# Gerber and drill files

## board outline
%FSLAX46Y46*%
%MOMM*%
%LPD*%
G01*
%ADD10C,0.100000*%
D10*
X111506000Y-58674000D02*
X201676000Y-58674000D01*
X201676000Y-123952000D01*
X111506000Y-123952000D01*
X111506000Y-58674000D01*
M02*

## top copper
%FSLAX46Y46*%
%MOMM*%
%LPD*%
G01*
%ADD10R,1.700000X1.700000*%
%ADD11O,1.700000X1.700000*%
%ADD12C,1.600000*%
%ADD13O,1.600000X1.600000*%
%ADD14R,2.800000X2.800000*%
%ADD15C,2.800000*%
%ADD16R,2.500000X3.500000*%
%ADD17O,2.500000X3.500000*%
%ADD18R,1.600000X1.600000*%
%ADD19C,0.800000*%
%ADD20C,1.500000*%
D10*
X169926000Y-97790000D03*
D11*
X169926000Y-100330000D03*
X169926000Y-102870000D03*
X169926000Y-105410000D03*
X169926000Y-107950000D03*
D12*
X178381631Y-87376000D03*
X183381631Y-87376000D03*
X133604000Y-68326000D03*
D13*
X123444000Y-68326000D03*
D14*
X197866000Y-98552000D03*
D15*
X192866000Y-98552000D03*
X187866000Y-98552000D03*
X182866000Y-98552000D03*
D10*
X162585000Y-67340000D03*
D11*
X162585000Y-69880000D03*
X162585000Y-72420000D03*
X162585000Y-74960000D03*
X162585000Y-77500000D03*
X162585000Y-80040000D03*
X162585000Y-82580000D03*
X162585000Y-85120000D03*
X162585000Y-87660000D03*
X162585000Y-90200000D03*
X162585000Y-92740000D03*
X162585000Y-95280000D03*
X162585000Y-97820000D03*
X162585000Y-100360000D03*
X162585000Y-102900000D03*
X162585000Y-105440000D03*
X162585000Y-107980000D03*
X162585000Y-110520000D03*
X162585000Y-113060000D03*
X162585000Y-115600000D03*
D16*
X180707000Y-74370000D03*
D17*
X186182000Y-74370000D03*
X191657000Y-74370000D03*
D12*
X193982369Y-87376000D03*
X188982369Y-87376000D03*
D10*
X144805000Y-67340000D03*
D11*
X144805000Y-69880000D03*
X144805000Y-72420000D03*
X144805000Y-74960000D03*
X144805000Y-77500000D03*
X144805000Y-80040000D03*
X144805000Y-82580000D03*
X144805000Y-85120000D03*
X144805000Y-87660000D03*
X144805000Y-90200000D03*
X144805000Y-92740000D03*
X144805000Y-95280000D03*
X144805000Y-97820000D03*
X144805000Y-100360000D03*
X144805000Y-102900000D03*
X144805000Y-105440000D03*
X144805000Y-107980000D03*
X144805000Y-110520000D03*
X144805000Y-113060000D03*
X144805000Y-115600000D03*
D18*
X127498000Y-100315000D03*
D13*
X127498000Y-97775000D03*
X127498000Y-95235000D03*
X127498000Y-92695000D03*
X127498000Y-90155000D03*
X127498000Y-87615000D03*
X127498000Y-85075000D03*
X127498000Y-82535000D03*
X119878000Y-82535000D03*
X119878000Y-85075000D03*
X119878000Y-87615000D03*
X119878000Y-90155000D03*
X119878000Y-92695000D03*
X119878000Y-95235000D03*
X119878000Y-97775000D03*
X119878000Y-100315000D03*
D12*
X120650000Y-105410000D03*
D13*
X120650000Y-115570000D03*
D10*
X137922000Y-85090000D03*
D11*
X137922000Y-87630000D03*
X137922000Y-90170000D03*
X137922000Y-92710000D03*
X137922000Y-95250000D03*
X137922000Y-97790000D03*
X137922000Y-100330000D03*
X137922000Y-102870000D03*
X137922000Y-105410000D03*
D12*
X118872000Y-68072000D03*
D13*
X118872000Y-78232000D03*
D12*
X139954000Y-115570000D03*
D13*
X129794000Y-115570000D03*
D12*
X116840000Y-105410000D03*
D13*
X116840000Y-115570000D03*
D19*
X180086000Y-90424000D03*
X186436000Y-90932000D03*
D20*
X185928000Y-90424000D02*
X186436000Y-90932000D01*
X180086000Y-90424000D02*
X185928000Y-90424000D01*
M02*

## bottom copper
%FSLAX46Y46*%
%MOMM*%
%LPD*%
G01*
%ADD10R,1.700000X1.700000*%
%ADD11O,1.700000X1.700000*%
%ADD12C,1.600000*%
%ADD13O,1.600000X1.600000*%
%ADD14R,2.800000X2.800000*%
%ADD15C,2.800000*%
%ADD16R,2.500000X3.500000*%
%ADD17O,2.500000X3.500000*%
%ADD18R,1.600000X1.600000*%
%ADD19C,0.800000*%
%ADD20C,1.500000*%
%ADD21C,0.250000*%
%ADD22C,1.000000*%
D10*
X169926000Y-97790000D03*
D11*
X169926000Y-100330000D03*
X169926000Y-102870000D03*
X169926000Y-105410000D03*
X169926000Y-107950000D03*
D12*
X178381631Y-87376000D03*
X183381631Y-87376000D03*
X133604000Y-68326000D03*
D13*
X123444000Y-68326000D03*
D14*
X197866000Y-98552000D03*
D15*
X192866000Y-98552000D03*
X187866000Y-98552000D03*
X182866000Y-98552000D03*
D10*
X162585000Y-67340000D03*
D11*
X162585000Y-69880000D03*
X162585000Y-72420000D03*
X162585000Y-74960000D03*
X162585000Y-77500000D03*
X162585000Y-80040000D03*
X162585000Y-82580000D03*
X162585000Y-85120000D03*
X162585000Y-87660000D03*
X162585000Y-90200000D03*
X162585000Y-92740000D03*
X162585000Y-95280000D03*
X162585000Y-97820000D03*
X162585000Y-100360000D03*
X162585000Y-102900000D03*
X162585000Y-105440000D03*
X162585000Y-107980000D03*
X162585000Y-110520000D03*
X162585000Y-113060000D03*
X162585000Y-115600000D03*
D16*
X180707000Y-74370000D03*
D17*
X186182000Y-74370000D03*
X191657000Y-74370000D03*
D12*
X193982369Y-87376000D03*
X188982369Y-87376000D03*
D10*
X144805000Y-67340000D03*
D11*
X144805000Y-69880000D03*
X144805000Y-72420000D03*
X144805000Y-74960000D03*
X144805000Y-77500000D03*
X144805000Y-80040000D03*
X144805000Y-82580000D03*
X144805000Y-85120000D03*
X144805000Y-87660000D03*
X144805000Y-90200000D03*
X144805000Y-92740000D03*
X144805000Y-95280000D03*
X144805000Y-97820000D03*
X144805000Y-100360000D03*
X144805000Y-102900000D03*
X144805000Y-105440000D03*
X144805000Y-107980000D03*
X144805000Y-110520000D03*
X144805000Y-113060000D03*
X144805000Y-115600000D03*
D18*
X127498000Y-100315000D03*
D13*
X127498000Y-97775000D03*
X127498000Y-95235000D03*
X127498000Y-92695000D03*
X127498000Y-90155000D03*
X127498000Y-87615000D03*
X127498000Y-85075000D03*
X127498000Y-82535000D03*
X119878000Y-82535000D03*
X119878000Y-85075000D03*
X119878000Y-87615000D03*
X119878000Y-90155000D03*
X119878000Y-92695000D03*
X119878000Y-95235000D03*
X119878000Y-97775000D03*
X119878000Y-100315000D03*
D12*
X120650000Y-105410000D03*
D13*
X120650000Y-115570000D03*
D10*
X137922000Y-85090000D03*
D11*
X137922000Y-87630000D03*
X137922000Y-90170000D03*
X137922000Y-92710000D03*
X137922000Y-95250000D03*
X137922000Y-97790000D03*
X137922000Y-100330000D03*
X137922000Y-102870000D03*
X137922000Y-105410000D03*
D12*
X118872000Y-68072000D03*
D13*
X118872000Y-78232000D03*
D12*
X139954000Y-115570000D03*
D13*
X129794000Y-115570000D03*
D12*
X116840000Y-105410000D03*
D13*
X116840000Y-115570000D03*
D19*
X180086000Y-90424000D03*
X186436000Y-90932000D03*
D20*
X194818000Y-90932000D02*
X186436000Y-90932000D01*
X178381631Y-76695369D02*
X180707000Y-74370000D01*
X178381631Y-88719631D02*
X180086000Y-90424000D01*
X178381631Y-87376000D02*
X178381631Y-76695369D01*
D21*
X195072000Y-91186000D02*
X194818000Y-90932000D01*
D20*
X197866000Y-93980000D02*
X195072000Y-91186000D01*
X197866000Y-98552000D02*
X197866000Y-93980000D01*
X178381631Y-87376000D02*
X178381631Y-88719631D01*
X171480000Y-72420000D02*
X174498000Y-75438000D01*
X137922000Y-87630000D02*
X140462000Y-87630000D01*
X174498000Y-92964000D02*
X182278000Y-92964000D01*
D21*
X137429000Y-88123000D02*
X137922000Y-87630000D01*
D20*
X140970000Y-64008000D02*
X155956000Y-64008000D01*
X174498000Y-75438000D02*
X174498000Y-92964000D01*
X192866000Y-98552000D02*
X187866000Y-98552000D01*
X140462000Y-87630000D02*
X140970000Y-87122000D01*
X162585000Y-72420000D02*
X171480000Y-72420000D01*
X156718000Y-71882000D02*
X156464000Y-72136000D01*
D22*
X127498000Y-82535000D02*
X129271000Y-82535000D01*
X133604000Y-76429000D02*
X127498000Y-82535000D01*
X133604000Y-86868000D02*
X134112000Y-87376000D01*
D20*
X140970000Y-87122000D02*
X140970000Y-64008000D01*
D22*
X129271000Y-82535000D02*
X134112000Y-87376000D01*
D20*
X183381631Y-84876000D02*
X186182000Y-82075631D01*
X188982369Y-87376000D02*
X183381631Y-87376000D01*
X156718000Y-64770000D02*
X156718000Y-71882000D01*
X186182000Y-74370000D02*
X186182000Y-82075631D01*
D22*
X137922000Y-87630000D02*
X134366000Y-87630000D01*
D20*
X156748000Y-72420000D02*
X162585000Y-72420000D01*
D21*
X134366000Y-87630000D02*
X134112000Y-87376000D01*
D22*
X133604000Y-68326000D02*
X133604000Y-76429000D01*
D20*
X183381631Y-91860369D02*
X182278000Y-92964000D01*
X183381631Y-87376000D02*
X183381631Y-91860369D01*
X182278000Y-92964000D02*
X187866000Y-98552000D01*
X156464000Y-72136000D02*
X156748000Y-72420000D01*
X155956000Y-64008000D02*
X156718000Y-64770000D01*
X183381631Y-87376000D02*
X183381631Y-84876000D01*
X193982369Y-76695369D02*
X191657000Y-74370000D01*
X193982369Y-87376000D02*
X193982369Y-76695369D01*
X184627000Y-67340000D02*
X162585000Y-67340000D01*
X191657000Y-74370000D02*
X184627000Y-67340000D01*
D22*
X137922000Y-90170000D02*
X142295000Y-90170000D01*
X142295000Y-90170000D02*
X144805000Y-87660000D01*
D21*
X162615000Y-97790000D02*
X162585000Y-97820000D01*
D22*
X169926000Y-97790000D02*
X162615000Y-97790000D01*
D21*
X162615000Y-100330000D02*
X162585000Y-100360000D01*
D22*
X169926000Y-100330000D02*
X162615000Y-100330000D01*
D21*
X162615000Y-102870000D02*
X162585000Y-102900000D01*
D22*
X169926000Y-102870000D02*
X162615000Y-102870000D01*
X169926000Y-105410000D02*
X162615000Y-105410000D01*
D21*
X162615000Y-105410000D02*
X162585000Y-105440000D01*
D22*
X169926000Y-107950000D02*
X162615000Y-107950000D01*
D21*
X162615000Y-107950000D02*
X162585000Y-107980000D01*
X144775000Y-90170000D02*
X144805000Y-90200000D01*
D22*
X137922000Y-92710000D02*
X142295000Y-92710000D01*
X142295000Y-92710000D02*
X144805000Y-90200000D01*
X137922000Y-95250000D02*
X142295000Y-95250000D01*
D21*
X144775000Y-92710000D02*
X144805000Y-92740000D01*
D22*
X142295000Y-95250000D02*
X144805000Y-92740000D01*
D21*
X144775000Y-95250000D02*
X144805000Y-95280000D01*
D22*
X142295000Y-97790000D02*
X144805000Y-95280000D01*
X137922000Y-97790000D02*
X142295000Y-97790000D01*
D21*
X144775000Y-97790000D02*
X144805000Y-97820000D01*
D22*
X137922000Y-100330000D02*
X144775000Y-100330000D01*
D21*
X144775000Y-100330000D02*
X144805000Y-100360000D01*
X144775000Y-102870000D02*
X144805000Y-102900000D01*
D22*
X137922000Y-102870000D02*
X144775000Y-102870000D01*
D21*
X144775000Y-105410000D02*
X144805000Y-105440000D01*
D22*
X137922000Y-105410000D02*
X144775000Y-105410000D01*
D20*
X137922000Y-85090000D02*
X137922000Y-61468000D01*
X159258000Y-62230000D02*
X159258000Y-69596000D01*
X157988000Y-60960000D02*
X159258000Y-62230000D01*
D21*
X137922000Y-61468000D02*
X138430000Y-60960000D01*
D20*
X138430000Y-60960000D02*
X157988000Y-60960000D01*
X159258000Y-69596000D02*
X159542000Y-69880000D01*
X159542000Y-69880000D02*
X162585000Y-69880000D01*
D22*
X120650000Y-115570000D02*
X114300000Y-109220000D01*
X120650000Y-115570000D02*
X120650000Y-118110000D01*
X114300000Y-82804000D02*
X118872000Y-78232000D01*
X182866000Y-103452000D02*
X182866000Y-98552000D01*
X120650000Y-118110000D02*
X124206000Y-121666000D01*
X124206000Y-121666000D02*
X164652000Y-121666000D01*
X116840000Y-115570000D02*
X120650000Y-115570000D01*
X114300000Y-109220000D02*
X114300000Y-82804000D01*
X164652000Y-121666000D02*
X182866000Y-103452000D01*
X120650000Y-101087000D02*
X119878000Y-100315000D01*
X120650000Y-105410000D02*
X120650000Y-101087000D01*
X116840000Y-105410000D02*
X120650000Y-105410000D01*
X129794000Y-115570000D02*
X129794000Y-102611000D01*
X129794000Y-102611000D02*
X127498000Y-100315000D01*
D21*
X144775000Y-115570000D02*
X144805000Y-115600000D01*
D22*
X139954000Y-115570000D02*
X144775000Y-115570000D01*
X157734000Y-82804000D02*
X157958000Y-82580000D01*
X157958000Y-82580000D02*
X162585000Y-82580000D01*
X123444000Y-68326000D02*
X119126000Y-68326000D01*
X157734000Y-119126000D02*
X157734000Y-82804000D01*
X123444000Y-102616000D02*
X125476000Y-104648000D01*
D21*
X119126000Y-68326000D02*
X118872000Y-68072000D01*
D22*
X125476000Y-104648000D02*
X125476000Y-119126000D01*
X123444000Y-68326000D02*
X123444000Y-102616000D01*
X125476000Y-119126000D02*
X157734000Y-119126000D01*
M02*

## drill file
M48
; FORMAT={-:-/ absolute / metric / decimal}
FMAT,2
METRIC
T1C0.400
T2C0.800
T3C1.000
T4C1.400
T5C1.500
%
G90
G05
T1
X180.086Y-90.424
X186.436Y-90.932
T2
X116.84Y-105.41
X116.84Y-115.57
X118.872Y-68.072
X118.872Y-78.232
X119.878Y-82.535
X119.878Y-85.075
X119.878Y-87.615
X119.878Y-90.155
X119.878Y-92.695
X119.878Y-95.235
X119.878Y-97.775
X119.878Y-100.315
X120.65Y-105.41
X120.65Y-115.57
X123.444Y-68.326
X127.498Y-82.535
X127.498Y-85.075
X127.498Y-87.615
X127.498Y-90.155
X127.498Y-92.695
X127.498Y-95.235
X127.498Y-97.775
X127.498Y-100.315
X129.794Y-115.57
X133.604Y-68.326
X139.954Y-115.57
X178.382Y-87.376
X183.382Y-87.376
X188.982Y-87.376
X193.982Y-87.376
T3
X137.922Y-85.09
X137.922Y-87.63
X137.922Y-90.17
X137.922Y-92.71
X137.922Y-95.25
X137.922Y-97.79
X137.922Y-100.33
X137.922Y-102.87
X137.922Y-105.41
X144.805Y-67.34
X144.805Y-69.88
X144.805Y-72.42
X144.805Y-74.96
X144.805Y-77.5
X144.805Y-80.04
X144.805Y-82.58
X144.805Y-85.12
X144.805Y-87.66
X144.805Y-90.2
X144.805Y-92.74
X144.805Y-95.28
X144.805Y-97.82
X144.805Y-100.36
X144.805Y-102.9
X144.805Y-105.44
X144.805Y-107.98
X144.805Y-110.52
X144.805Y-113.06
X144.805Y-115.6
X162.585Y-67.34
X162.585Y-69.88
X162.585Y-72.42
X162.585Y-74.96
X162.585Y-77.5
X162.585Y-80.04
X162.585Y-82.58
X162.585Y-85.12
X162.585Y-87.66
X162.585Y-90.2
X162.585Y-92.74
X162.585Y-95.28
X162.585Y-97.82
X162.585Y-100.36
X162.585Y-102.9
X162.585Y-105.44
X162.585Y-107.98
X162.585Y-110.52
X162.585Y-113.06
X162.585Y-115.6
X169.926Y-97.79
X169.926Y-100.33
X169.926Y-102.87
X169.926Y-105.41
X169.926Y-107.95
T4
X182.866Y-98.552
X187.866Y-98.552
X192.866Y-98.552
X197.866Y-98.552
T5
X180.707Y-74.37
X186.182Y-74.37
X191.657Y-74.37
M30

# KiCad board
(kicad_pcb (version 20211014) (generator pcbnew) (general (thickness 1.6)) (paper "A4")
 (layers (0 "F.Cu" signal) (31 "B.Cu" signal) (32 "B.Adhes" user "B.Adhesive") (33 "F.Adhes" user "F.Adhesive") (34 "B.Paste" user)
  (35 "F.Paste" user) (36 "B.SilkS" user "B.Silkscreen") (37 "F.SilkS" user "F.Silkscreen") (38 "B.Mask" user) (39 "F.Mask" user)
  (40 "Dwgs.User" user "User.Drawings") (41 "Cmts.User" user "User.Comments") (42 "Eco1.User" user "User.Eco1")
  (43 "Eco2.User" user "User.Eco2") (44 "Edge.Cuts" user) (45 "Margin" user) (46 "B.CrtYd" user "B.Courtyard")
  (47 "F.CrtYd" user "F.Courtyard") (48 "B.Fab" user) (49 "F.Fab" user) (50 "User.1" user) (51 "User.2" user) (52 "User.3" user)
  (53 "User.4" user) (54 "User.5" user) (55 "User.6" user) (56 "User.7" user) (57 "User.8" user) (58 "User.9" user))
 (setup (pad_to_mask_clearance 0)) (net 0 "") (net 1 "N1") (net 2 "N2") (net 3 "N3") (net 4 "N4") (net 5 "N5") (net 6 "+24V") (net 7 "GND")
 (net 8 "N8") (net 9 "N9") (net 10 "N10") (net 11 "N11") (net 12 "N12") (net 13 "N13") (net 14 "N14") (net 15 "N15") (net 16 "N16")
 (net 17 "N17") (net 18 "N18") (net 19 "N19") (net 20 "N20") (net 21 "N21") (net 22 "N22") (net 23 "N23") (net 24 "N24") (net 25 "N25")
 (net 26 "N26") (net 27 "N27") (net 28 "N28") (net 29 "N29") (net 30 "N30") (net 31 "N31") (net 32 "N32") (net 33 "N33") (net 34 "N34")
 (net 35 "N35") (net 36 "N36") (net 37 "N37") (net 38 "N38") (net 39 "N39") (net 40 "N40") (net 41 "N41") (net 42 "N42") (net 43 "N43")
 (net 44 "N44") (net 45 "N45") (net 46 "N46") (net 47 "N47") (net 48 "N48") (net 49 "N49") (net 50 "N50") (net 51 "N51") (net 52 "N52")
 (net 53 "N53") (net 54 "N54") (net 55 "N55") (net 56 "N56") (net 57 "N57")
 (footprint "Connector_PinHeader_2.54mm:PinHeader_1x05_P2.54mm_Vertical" (layer "F.Cu") (at 169.926 97.79)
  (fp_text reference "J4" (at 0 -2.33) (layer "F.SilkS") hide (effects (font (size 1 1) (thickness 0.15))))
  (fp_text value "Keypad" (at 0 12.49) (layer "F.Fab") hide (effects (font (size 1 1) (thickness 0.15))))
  (pad "1" thru_hole rect (at 0 0) (size 1.7 1.7) (drill 1) (layers *.Cu *.Mask) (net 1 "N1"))
  (pad "2" thru_hole oval (at 0 2.54) (size 1.7 1.7) (drill 1) (layers *.Cu *.Mask) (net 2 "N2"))
  (pad "3" thru_hole oval (at 0 5.08) (size 1.7 1.7) (drill 1) (layers *.Cu *.Mask) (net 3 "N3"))
  (pad "4" thru_hole oval (at 0 7.62) (size 1.7 1.7) (drill 1) (layers *.Cu *.Mask) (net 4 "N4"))
  (pad "5" thru_hole oval (at 0 10.16) (size 1.7 1.7) (drill 1) (layers *.Cu *.Mask) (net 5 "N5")))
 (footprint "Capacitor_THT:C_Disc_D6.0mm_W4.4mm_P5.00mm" (layer "F.Cu") (at 178.381631 87.376)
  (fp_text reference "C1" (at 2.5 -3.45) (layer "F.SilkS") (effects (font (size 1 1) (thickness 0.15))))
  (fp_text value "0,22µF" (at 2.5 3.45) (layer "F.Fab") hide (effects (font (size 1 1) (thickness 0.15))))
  (pad "1" thru_hole circle (at 0 0) (size 1.6 1.6) (drill 0.8) (layers *.Cu *.Mask) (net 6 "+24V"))
  (pad "2" thru_hole circle (at 5 0) (size 1.6 1.6) (drill 0.8) (layers *.Cu *.Mask) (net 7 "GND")))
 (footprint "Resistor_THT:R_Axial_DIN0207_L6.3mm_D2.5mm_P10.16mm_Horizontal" (layer "F.Cu") (at 133.604 68.326 180)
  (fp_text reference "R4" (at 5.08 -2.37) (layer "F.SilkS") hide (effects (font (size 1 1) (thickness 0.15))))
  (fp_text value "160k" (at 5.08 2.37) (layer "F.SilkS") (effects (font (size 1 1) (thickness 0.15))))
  (pad "1" thru_hole circle (at 0 0 180) (size 1.6 1.6) (drill 0.8) (layers *.Cu *.Mask) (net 7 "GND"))
  (pad "2" thru_hole oval (at 10.16 0 180) (size 1.6 1.6) (drill 0.8) (layers *.Cu *.Mask) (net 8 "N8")))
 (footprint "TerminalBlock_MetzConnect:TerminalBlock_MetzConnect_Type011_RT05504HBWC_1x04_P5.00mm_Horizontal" (layer "F.Cu")
  (at 197.866 98.552 180)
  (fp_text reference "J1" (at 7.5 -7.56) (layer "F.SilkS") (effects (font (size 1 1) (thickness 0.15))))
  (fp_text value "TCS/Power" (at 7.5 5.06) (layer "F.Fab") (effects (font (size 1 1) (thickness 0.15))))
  (pad "1" thru_hole rect (at 0 0 180) (size 2.8 2.8) (drill 1.4) (layers *.Cu *.Mask) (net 6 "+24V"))
  (pad "2" thru_hole circle (at 5 0 180) (size 2.8 2.8) (drill 1.4) (layers *.Cu *.Mask) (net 7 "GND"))
  (pad "3" thru_hole circle (at 10 0 180) (size 2.8 2.8) (drill 1.4) (layers *.Cu *.Mask) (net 7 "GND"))
  (pad "4" thru_hole circle (at 15 0 180) (size 2.8 2.8) (drill 1.4) (layers *.Cu *.Mask) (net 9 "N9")))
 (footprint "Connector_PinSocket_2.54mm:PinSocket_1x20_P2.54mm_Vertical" (layer "F.Cu") (at 162.585 67.34)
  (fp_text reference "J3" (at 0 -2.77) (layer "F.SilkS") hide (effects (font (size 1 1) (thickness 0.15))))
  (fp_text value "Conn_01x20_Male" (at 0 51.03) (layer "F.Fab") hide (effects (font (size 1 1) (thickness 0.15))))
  (pad "1" thru_hole rect (at 0 0) (size 1.7 1.7) (drill 1) (layers *.Cu *.Mask) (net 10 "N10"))
  (pad "2" thru_hole oval (at 0 2.54) (size 1.7 1.7) (drill 1) (layers *.Cu *.Mask) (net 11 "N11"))
  (pad "3" thru_hole oval (at 0 5.08) (size 1.7 1.7) (drill 1) (layers *.Cu *.Mask) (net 7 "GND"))
  (pad "4" thru_hole oval (at 0 7.62) (size 1.7 1.7) (drill 1) (layers *.Cu *.Mask) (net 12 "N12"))
  (pad "5" thru_hole oval (at 0 10.16) (size 1.7 1.7) (drill 1) (layers *.Cu *.Mask) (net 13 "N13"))
  (pad "6" thru_hole oval (at 0 12.7) (size 1.7 1.7) (drill 1) (layers *.Cu *.Mask) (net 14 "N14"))
  (pad "7" thru_hole oval (at 0 15.24) (size 1.7 1.7) (drill 1) (layers *.Cu *.Mask) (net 8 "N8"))
  (pad "8" thru_hole oval (at 0 17.78) (size 1.7 1.7) (drill 1) (layers *.Cu *.Mask) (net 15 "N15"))
  (pad "9" thru_hole oval (at 0 20.32) (size 1.7 1.7) (drill 1) (layers *.Cu *.Mask) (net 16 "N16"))
  (pad "10" thru_hole oval (at 0 22.86) (size 1.7 1.7) (drill 1) (layers *.Cu *.Mask) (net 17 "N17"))
  (pad "11" thru_hole oval (at 0 25.4) (size 1.7 1.7) (drill 1) (layers *.Cu *.Mask) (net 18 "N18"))
  (pad "12" thru_hole oval (at 0 27.94) (size 1.7 1.7) (drill 1) (layers *.Cu *.Mask) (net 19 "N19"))
  (pad "13" thru_hole oval (at 0 30.48) (size 1.7 1.7) (drill 1) (layers *.Cu *.Mask) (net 1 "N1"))
  (pad "14" thru_hole oval (at 0 33.02) (size 1.7 1.7) (drill 1) (layers *.Cu *.Mask) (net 2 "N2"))
  (pad "15" thru_hole oval (at 0 35.56) (size 1.7 1.7) (drill 1) (layers *.Cu *.Mask) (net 3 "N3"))
  (pad "16" thru_hole oval (at 0 38.1) (size 1.7 1.7) (drill 1) (layers *.Cu *.Mask) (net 4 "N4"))
  (pad "17" thru_hole oval (at 0 40.64) (size 1.7 1.7) (drill 1) (layers *.Cu *.Mask) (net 5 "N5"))
  (pad "18" thru_hole oval (at 0 43.18) (size 1.7 1.7) (drill 1) (layers *.Cu *.Mask) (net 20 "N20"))
  (pad "19" thru_hole oval (at 0 45.72) (size 1.7 1.7) (drill 1) (layers *.Cu *.Mask) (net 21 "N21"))
  (pad "20" thru_hole oval (at 0 48.26) (size 1.7 1.7) (drill 1) (layers *.Cu *.Mask) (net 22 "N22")))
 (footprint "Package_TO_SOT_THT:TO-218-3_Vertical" (layer "F.Cu") (at 180.707 74.37)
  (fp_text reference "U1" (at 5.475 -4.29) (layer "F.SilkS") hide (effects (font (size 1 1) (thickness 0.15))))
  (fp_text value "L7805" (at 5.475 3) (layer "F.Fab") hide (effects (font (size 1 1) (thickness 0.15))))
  (pad "1" thru_hole rect (at 0 0) (size 2.5 3.5) (drill 1.5) (layers *.Cu *.Mask) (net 6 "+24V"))
  (pad "2" thru_hole oval (at 5.475 0) (size 2.5 3.5) (drill 1.5) (layers *.Cu *.Mask) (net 7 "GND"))
  (pad "3" thru_hole oval (at 10.95 0) (size 2.5 3.5) (drill 1.5) (layers *.Cu *.Mask) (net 10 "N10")))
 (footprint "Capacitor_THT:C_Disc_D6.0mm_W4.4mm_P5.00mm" (layer "F.Cu") (at 193.982369 87.376 180)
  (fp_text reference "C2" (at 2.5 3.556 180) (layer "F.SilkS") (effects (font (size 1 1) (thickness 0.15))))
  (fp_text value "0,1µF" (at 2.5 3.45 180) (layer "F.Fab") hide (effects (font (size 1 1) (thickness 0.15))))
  (pad "1" thru_hole circle (at 0 0 180) (size 1.6 1.6) (drill 0.8) (layers *.Cu *.Mask) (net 10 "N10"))
  (pad "2" thru_hole circle (at 5 0 180) (size 1.6 1.6) (drill 0.8) (layers *.Cu *.Mask) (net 7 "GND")))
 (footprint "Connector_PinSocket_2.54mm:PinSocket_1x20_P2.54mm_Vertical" (layer "F.Cu") (at 144.805 67.34)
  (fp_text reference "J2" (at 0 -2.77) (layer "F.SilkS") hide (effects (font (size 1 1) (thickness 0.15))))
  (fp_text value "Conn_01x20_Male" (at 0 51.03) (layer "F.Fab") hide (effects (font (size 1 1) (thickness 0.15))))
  (pad "1" thru_hole rect (at 0 0) (size 1.7 1.7) (drill 1) (layers *.Cu *.Mask) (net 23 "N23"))
  (pad "2" thru_hole oval (at 0 2.54) (size 1.7 1.7) (drill 1) (layers *.Cu *.Mask) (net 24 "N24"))
  (pad "3" thru_hole oval (at 0 5.08) (size 1.7 1.7) (drill 1) (layers *.Cu *.Mask) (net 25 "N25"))
  (pad "4" thru_hole oval (at 0 7.62) (size 1.7 1.7) (drill 1) (layers *.Cu *.Mask) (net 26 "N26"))
  (pad "5" thru_hole oval (at 0 10.16) (size 1.7 1.7) (drill 1) (layers *.Cu *.Mask) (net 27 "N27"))
  (pad "6" thru_hole oval (at 0 12.7) (size 1.7 1.7) (drill 1) (layers *.Cu *.Mask) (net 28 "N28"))
  (pad "7" thru_hole oval (at 0 15.24) (size 1.7 1.7) (drill 1) (layers *.Cu *.Mask) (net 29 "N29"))
  (pad "8" thru_hole oval (at 0 17.78) (size 1.7 1.7) (drill 1) (layers *.Cu *.Mask) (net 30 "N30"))
  (pad "9" thru_hole oval (at 0 20.32) (size 1.7 1.7) (drill 1) (layers *.Cu *.Mask) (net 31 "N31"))
  (pad "10" thru_hole oval (at 0 22.86) (size 1.7 1.7) (drill 1) (layers *.Cu *.Mask) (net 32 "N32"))
  (pad "11" thru_hole oval (at 0 25.4) (size 1.7 1.7) (drill 1) (layers *.Cu *.Mask) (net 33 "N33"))
  (pad "12" thru_hole oval (at 0 27.94) (size 1.7 1.7) (drill 1) (layers *.Cu *.Mask) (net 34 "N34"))
  (pad "13" thru_hole oval (at 0 30.48) (size 1.7 1.7) (drill 1) (layers *.Cu *.Mask) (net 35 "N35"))
  (pad "14" thru_hole oval (at 0 33.02) (size 1.7 1.7) (drill 1) (layers *.Cu *.Mask) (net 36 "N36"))
  (pad "15" thru_hole oval (at 0 35.56) (size 1.7 1.7) (drill 1) (layers *.Cu *.Mask) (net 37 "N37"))
  (pad "16" thru_hole oval (at 0 38.1) (size 1.7 1.7) (drill 1) (layers *.Cu *.Mask) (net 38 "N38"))
  (pad "17" thru_hole oval (at 0 40.64) (size 1.7 1.7) (drill 1) (layers *.Cu *.Mask) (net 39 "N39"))
  (pad "18" thru_hole oval (at 0 43.18) (size 1.7 1.7) (drill 1) (layers *.Cu *.Mask) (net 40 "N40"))
  (pad "19" thru_hole oval (at 0 45.72) (size 1.7 1.7) (drill 1) (layers *.Cu *.Mask) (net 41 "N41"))
  (pad "20" thru_hole oval (at 0 48.26) (size 1.7 1.7) (drill 1) (layers *.Cu *.Mask) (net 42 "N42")))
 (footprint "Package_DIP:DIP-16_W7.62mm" (layer "F.Cu") (at 127.498 100.315 180)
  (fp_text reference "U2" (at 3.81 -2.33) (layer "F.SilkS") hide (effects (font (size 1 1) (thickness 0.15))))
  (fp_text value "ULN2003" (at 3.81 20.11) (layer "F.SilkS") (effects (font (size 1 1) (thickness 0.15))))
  (pad "1" thru_hole rect (at 0 0 180) (size 1.6 1.6) (drill 0.8) (layers *.Cu *.Mask) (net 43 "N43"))
  (pad "2" thru_hole oval (at 0 2.54 180) (size 1.6 1.6) (drill 0.8) (layers *.Cu *.Mask) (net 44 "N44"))
  (pad "3" thru_hole oval (at 0 5.08 180) (size 1.6 1.6) (drill 0.8) (layers *.Cu *.Mask) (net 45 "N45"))
  (pad "4" thru_hole oval (at 0 7.62 180) (size 1.6 1.6) (drill 0.8) (layers *.Cu *.Mask) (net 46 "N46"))
  (pad "5" thru_hole oval (at 0 10.16 180) (size 1.6 1.6) (drill 0.8) (layers *.Cu *.Mask) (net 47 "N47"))
  (pad "6" thru_hole oval (at 0 12.7 180) (size 1.6 1.6) (drill 0.8) (layers *.Cu *.Mask) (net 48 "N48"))
  (pad "7" thru_hole oval (at 0 15.24 180) (size 1.6 1.6) (drill 0.8) (layers *.Cu *.Mask) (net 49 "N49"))
  (pad "8" thru_hole oval (at 0 17.78 180) (size 1.6 1.6) (drill 0.8) (layers *.Cu *.Mask) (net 7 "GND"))
  (pad "9" thru_hole oval (at 7.62 17.78 180) (size 1.6 1.6) (drill 0.8) (layers *.Cu *.Mask) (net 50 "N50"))
  (pad "10" thru_hole oval (at 7.62 15.24 180) (size 1.6 1.6) (drill 0.8) (layers *.Cu *.Mask) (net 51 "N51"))
  (pad "11" thru_hole oval (at 7.62 12.7 180) (size 1.6 1.6) (drill 0.8) (layers *.Cu *.Mask) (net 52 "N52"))
  (pad "12" thru_hole oval (at 7.62 10.16 180) (size 1.6 1.6) (drill 0.8) (layers *.Cu *.Mask) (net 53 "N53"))
  (pad "13" thru_hole oval (at 7.62 7.62 180) (size 1.6 1.6) (drill 0.8) (layers *.Cu *.Mask) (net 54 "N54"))
  (pad "14" thru_hole oval (at 7.62 5.08 180) (size 1.6 1.6) (drill 0.8) (layers *.Cu *.Mask) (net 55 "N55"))
  (pad "15" thru_hole oval (at 7.62 2.54 180) (size 1.6 1.6) (drill 0.8) (layers *.Cu *.Mask) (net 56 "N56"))
  (pad "16" thru_hole oval (at 7.62 0 180) (size 1.6 1.6) (drill 0.8) (layers *.Cu *.Mask) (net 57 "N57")))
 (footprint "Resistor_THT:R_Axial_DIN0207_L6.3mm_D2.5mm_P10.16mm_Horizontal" (layer "F.Cu") (at 120.65 105.41 -90)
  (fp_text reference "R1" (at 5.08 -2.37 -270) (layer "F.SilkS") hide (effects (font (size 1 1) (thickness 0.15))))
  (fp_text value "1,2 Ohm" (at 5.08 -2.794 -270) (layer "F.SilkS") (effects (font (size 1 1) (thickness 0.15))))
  (pad "1" thru_hole circle (at 0 0 270) (size 1.6 1.6) (drill 0.8) (layers *.Cu *.Mask) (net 57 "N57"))
  (pad "2" thru_hole oval (at 10.16 0 270) (size 1.6 1.6) (drill 0.8) (layers *.Cu *.Mask) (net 9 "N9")))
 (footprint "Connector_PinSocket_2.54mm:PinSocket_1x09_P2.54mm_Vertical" (layer "F.Cu") (at 137.922 85.09)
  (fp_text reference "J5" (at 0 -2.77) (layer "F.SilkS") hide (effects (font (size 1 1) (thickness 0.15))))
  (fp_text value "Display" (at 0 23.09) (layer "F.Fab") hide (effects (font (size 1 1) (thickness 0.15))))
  (pad "1" thru_hole rect (at 0 0) (size 1.7 1.7) (drill 1) (layers *.Cu *.Mask) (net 11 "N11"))
  (pad "2" thru_hole oval (at 0 2.54) (size 1.7 1.7) (drill 1) (layers *.Cu *.Mask) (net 7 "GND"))
  (pad "3" thru_hole oval (at 0 5.08) (size 1.7 1.7) (drill 1) (layers *.Cu *.Mask) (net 31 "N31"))
  (pad "4" thru_hole oval (at 0 7.62) (size 1.7 1.7) (drill 1) (layers *.Cu *.Mask) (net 32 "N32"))
  (pad "5" thru_hole oval (at 0 10.16) (size 1.7 1.7) (drill 1) (layers *.Cu *.Mask) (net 33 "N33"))
  (pad "6" thru_hole oval (at 0 12.7) (size 1.7 1.7) (drill 1) (layers *.Cu *.Mask) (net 34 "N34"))
  (pad "7" thru_hole oval (at 0 15.24) (size 1.7 1.7) (drill 1) (layers *.Cu *.Mask) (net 36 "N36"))
  (pad "8" thru_hole oval (at 0 17.78) (size 1.7 1.7) (drill 1) (layers *.Cu *.Mask) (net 37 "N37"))
  (pad "9" thru_hole oval (at 0 20.32) (size 1.7 1.7) (drill 1) (layers *.Cu *.Mask) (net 38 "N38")))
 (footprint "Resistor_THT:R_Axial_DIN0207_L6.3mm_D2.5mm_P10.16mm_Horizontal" (layer "F.Cu") (at 118.872 68.072 -90)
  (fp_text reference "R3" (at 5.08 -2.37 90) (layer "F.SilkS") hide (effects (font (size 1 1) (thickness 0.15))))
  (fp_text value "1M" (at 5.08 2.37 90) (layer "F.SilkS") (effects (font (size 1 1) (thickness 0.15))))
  (pad "1" thru_hole circle (at 0 0 270) (size 1.6 1.6) (drill 0.8) (layers *.Cu *.Mask) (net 8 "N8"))
  (pad "2" thru_hole oval (at 10.16 0 270) (size 1.6 1.6) (drill 0.8) (layers *.Cu *.Mask) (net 9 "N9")))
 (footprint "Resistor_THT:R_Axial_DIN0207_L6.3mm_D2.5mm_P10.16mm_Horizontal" (layer "F.Cu") (at 139.954 115.57 180)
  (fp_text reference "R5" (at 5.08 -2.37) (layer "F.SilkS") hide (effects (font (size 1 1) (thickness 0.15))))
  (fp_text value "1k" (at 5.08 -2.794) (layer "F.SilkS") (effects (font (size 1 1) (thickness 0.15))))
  (pad "1" thru_hole circle (at 0 0 180) (size 1.6 1.6) (drill 0.8) (layers *.Cu *.Mask) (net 42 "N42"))
  (pad "2" thru_hole oval (at 10.16 0 180) (size 1.6 1.6) (drill 0.8) (layers *.Cu *.Mask) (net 43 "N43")))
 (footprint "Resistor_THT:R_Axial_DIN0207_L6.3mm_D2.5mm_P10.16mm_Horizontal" (layer "F.Cu") (at 116.84 105.41 -90)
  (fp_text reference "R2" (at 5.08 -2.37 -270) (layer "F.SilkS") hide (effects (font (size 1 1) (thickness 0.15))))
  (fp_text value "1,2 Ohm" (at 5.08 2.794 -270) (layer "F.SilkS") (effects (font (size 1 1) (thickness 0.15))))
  (pad "1" thru_hole circle (at 0 0 270) (size 1.6 1.6) (drill 0.8) (layers *.Cu *.Mask) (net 57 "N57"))
  (pad "2" thru_hole oval (at 10.16 0 270) (size 1.6 1.6) (drill 0.8) (layers *.Cu *.Mask) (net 9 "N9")))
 (gr_rect (start 111.506 58.674) (end 201.676 123.952) (layer "Edge.Cuts") (width 0.1) (fill none))
 (segment (start 185.928 90.424) (end 186.436 90.932) (width 1.5) (layer "F.Cu") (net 6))
 (segment (start 180.086 90.424) (end 185.928 90.424) (width 1.5) (layer "F.Cu") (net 6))
 (via (at 180.086 90.424) (size 0.8) (drill 0.4) (layers "F.Cu" "B.Cu") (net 6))
 (via (at 186.436 90.932) (size 0.8) (drill 0.4) (layers "F.Cu" "B.Cu") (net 6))
 (segment (start 194.818 90.932) (end 186.436 90.932) (width 1.5) (layer "B.Cu") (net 6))
 (segment (start 178.381631 76.695369) (end 180.707 74.37) (width 1.5) (layer "B.Cu") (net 6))
 (segment (start 178.381631 88.719631) (end 180.086 90.424) (width 1.5) (layer "B.Cu") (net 6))
 (segment (start 178.381631 87.376) (end 178.381631 76.695369) (width 1.5) (layer "B.Cu") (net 6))
 (segment (start 195.072 91.186) (end 194.818 90.932) (width 0.25) (layer "B.Cu") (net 6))
 (segment (start 197.866 93.98) (end 195.072 91.186) (width 1.5) (layer "B.Cu") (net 6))
 (segment (start 197.866 98.552) (end 197.866 93.98) (width 1.5) (layer "B.Cu") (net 6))
 (segment (start 178.381631 87.376) (end 178.381631 88.719631) (width 1.5) (layer "B.Cu") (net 6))
 (segment (start 171.48 72.42) (end 174.498 75.438) (width 1.5) (layer "B.Cu") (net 7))
 (segment (start 137.922 87.63) (end 140.462 87.63) (width 1.5) (layer "B.Cu") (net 7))
 (segment (start 174.498 92.964) (end 182.278 92.964) (width 1.5) (layer "B.Cu") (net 7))
 (segment (start 137.429 88.123) (end 137.922 87.63) (width 0.25) (layer "B.Cu") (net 7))
 (segment (start 140.97 64.008) (end 155.956 64.008) (width 1.5) (layer "B.Cu") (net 7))
 (segment (start 174.498 75.438) (end 174.498 92.964) (width 1.5) (layer "B.Cu") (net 7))
 (segment (start 192.866 98.552) (end 187.866 98.552) (width 1.5) (layer "B.Cu") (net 7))
 (segment (start 140.462 87.63) (end 140.97 87.122) (width 1.5) (layer "B.Cu") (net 7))
 (segment (start 162.585 72.42) (end 171.48 72.42) (width 1.5) (layer "B.Cu") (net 7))
 (segment (start 156.718 71.882) (end 156.464 72.136) (width 1.5) (layer "B.Cu") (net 7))
 (segment (start 127.498 82.535) (end 129.271 82.535) (width 1) (layer "B.Cu") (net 7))
 (segment (start 133.604 76.429) (end 127.498 82.535) (width 1) (layer "B.Cu") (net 7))
 (segment (start 133.604 86.868) (end 134.112 87.376) (width 1) (layer "B.Cu") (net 7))
 (segment (start 140.97 87.122) (end 140.97 64.008) (width 1.5) (layer "B.Cu") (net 7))
 (segment (start 129.271 82.535) (end 134.112 87.376) (width 1) (layer "B.Cu") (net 7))
 (segment (start 183.381631 84.876) (end 186.182 82.075631) (width 1.5) (layer "B.Cu") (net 7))
 (segment (start 188.982369 87.376) (end 183.381631 87.376) (width 1.5) (layer "B.Cu") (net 7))
 (segment (start 156.718 64.77) (end 156.718 71.882) (width 1.5) (layer "B.Cu") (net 7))
 (segment (start 186.182 74.37) (end 186.182 82.075631) (width 1.5) (layer "B.Cu") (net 7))
 (segment (start 137.922 87.63) (end 134.366 87.63) (width 1) (layer "B.Cu") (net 7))
 (segment (start 156.748 72.42) (end 162.585 72.42) (width 1.5) (layer "B.Cu") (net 7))
 (segment (start 134.366 87.63) (end 134.112 87.376) (width 0.25) (layer "B.Cu") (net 7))
 (segment (start 133.604 68.326) (end 133.604 76.429) (width 1) (layer "B.Cu") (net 7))
 (segment (start 183.381631 91.860369) (end 182.278 92.964) (width 1.5) (layer "B.Cu") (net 7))
 (segment (start 183.381631 87.376) (end 183.381631 91.860369) (width 1.5) (layer "B.Cu") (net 7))
 (segment (start 182.278 92.964) (end 187.866 98.552) (width 1.5) (layer "B.Cu") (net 7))
 (segment (start 156.464 72.136) (end 156.748 72.42) (width 1.5) (layer "B.Cu") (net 7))
 (segment (start 155.956 64.008) (end 156.718 64.77) (width 1.5) (layer "B.Cu") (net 7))
 (segment (start 183.381631 87.376) (end 183.381631 84.876) (width 1.5) (layer "B.Cu") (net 7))
 (segment (start 193.982369 76.695369) (end 191.657 74.37) (width 1.5) (layer "B.Cu") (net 10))
 (segment (start 193.982369 87.376) (end 193.982369 76.695369) (width 1.5) (layer "B.Cu") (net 10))
 (segment (start 184.627 67.34) (end 162.585 67.34) (width 1.5) (layer "B.Cu") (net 10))
 (segment (start 191.657 74.37) (end 184.627 67.34) (width 1.5) (layer "B.Cu") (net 10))
 (segment (start 137.922 90.17) (end 142.295 90.17) (width 1) (layer "B.Cu") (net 31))
 (segment (start 142.295 90.17) (end 144.805 87.66) (width 1) (layer "B.Cu") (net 31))
 (segment (start 162.615 97.79) (end 162.585 97.82) (width 0.25) (layer "B.Cu") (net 1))
 (segment (start 169.926 97.79) (end 162.615 97.79) (width 1) (layer "B.Cu") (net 1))
 (segment (start 162.615 100.33) (end 162.585 100.36) (width 0.25) (layer "B.Cu") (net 2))
 (segment (start 169.926 100.33) (end 162.615 100.33) (width 1) (layer "B.Cu") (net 2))
 (segment (start 162.615 102.87) (end 162.585 102.9) (width 0.25) (layer "B.Cu") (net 3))
 (segment (start 169.926 102.87) (end 162.615 102.87) (width 1) (layer "B.Cu") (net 3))
 (segment (start 169.926 105.41) (end 162.615 105.41) (width 1) (layer "B.Cu") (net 4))
 (segment (start 162.615 105.41) (end 162.585 105.44) (width 0.25) (layer "B.Cu") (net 4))
 (segment (start 169.926 107.95) (end 162.615 107.95) (width 1) (layer "B.Cu") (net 5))
 (segment (start 162.615 107.95) (end 162.585 107.98) (width 0.25) (layer "B.Cu") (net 5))
 (segment (start 144.775 90.17) (end 144.805 90.2) (width 0.25) (layer "B.Cu") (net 32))
 (segment (start 137.922 92.71) (end 142.295 92.71) (width 1) (layer "B.Cu") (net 32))
 (segment (start 142.295 92.71) (end 144.805 90.2) (width 1) (layer "B.Cu") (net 32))
 (segment (start 137.922 95.25) (end 142.295 95.25) (width 1) (layer "B.Cu") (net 33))
 (segment (start 144.775 92.71) (end 144.805 92.74) (width 0.25) (layer "B.Cu") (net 33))
 (segment (start 142.295 95.25) (end 144.805 92.74) (width 1) (layer "B.Cu") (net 33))
 (segment (start 144.775 95.25) (end 144.805 95.28) (width 0.25) (layer "B.Cu") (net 34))
 (segment (start 142.295 97.79) (end 144.805 95.28) (width 1) (layer "B.Cu") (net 34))
 (segment (start 137.922 97.79) (end 142.295 97.79) (width 1) (layer "B.Cu") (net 34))
 (segment (start 144.775 97.79) (end 144.805 97.82) (width 0.25) (layer "B.Cu") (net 35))
 (segment (start 137.922 100.33) (end 144.775 100.33) (width 1) (layer "B.Cu") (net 36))
 (segment (start 144.775 100.33) (end 144.805 100.36) (width 0.25) (layer "B.Cu") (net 36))
 (segment (start 144.775 102.87) (end 144.805 102.9) (width 0.25) (layer "B.Cu") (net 37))
 (segment (start 137.922 102.87) (end 144.775 102.87) (width 1) (layer "B.Cu") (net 37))
 (segment (start 144.775 105.41) (end 144.805 105.44) (width 0.25) (layer "B.Cu") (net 38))
 (segment (start 137.922 105.41) (end 144.775 105.41) (width 1) (layer "B.Cu") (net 38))
 (segment (start 137.922 85.09) (end 137.922 61.468) (width 1.5) (layer "B.Cu") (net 11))
 (segment (start 159.258 62.23) (end 159.258 69.596) (width 1.5) (layer "B.Cu") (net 11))
 (segment (start 157.988 60.96) (end 159.258 62.23) (width 1.5) (layer "B.Cu") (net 11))
 (segment (start 137.922 61.468) (end 138.43 60.96) (width 0.25) (layer "B.Cu") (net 11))
 (segment (start 138.43 60.96) (end 157.988 60.96) (width 1.5) (layer "B.Cu") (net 11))
 (segment (start 159.258 69.596) (end 159.542 69.88) (width 1.5) (layer "B.Cu") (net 11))
 (segment (start 159.542 69.88) (end 162.585 69.88) (width 1.5) (layer "B.Cu") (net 11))
 (segment (start 120.65 115.57) (end 114.3 109.22) (width 1) (layer "B.Cu") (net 9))
 (segment (start 120.65 115.57) (end 120.65 118.11) (width 1) (layer "B.Cu") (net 9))
 (segment (start 114.3 82.804) (end 118.872 78.232) (width 1) (layer "B.Cu") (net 9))
 (segment (start 182.866 103.452) (end 182.866 98.552) (width 1) (layer "B.Cu") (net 9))
 (segment (start 120.65 118.11) (end 124.206 121.666) (width 1) (layer "B.Cu") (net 9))
 (segment (start 124.206 121.666) (end 164.652 121.666) (width 1) (layer "B.Cu") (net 9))
 (segment (start 116.84 115.57) (end 120.65 115.57) (width 1) (layer "B.Cu") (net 9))
 (segment (start 114.3 109.22) (end 114.3 82.804) (width 1) (layer "B.Cu") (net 9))
 (segment (start 164.652 121.666) (end 182.866 103.452) (width 1) (layer "B.Cu") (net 9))
 (segment (start 120.65 101.087) (end 119.878 100.315) (width 1) (layer "B.Cu") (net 57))
 (segment (start 120.65 105.41) (end 120.65 101.087) (width 1) (layer "B.Cu") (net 57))
 (segment (start 116.84 105.41) (end 120.65 105.41) (width 1) (layer "B.Cu") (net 57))
 (segment (start 129.794 115.57) (end 129.794 102.611) (width 1) (layer "B.Cu") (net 43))
 (segment (start 129.794 102.611) (end 127.498 100.315) (width 1) (layer "B.Cu") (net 43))
 (segment (start 144.775 115.57) (end 144.805 115.6) (width 0.25) (layer "B.Cu") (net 42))
 (segment (start 139.954 115.57) (end 144.775 115.57) (width 1) (layer "B.Cu") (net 42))
 (segment (start 157.734 82.804) (end 157.958 82.58) (width 1) (layer "B.Cu") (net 8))
 (segment (start 157.958 82.58) (end 162.585 82.58) (width 1) (layer "B.Cu") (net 8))
 (segment (start 123.444 68.326) (end 119.126 68.326) (width 1) (layer "B.Cu") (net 8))
 (segment (start 157.734 119.126) (end 157.734 82.804) (width 1) (layer "B.Cu") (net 8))
 (segment (start 123.444 102.616) (end 125.476 104.648) (width 1) (layer "B.Cu") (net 8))
 (segment (start 119.126 68.326) (end 118.872 68.072) (width 0.25) (layer "B.Cu") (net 8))
 (segment (start 125.476 104.648) (end 125.476 119.126) (width 1) (layer "B.Cu") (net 8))
 (segment (start 123.444 68.326) (end 123.444 102.616) (width 1) (layer "B.Cu") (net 8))
 (segment (start 125.476 119.126) (end 157.734 119.126) (width 1) (layer "B.Cu") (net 8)))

